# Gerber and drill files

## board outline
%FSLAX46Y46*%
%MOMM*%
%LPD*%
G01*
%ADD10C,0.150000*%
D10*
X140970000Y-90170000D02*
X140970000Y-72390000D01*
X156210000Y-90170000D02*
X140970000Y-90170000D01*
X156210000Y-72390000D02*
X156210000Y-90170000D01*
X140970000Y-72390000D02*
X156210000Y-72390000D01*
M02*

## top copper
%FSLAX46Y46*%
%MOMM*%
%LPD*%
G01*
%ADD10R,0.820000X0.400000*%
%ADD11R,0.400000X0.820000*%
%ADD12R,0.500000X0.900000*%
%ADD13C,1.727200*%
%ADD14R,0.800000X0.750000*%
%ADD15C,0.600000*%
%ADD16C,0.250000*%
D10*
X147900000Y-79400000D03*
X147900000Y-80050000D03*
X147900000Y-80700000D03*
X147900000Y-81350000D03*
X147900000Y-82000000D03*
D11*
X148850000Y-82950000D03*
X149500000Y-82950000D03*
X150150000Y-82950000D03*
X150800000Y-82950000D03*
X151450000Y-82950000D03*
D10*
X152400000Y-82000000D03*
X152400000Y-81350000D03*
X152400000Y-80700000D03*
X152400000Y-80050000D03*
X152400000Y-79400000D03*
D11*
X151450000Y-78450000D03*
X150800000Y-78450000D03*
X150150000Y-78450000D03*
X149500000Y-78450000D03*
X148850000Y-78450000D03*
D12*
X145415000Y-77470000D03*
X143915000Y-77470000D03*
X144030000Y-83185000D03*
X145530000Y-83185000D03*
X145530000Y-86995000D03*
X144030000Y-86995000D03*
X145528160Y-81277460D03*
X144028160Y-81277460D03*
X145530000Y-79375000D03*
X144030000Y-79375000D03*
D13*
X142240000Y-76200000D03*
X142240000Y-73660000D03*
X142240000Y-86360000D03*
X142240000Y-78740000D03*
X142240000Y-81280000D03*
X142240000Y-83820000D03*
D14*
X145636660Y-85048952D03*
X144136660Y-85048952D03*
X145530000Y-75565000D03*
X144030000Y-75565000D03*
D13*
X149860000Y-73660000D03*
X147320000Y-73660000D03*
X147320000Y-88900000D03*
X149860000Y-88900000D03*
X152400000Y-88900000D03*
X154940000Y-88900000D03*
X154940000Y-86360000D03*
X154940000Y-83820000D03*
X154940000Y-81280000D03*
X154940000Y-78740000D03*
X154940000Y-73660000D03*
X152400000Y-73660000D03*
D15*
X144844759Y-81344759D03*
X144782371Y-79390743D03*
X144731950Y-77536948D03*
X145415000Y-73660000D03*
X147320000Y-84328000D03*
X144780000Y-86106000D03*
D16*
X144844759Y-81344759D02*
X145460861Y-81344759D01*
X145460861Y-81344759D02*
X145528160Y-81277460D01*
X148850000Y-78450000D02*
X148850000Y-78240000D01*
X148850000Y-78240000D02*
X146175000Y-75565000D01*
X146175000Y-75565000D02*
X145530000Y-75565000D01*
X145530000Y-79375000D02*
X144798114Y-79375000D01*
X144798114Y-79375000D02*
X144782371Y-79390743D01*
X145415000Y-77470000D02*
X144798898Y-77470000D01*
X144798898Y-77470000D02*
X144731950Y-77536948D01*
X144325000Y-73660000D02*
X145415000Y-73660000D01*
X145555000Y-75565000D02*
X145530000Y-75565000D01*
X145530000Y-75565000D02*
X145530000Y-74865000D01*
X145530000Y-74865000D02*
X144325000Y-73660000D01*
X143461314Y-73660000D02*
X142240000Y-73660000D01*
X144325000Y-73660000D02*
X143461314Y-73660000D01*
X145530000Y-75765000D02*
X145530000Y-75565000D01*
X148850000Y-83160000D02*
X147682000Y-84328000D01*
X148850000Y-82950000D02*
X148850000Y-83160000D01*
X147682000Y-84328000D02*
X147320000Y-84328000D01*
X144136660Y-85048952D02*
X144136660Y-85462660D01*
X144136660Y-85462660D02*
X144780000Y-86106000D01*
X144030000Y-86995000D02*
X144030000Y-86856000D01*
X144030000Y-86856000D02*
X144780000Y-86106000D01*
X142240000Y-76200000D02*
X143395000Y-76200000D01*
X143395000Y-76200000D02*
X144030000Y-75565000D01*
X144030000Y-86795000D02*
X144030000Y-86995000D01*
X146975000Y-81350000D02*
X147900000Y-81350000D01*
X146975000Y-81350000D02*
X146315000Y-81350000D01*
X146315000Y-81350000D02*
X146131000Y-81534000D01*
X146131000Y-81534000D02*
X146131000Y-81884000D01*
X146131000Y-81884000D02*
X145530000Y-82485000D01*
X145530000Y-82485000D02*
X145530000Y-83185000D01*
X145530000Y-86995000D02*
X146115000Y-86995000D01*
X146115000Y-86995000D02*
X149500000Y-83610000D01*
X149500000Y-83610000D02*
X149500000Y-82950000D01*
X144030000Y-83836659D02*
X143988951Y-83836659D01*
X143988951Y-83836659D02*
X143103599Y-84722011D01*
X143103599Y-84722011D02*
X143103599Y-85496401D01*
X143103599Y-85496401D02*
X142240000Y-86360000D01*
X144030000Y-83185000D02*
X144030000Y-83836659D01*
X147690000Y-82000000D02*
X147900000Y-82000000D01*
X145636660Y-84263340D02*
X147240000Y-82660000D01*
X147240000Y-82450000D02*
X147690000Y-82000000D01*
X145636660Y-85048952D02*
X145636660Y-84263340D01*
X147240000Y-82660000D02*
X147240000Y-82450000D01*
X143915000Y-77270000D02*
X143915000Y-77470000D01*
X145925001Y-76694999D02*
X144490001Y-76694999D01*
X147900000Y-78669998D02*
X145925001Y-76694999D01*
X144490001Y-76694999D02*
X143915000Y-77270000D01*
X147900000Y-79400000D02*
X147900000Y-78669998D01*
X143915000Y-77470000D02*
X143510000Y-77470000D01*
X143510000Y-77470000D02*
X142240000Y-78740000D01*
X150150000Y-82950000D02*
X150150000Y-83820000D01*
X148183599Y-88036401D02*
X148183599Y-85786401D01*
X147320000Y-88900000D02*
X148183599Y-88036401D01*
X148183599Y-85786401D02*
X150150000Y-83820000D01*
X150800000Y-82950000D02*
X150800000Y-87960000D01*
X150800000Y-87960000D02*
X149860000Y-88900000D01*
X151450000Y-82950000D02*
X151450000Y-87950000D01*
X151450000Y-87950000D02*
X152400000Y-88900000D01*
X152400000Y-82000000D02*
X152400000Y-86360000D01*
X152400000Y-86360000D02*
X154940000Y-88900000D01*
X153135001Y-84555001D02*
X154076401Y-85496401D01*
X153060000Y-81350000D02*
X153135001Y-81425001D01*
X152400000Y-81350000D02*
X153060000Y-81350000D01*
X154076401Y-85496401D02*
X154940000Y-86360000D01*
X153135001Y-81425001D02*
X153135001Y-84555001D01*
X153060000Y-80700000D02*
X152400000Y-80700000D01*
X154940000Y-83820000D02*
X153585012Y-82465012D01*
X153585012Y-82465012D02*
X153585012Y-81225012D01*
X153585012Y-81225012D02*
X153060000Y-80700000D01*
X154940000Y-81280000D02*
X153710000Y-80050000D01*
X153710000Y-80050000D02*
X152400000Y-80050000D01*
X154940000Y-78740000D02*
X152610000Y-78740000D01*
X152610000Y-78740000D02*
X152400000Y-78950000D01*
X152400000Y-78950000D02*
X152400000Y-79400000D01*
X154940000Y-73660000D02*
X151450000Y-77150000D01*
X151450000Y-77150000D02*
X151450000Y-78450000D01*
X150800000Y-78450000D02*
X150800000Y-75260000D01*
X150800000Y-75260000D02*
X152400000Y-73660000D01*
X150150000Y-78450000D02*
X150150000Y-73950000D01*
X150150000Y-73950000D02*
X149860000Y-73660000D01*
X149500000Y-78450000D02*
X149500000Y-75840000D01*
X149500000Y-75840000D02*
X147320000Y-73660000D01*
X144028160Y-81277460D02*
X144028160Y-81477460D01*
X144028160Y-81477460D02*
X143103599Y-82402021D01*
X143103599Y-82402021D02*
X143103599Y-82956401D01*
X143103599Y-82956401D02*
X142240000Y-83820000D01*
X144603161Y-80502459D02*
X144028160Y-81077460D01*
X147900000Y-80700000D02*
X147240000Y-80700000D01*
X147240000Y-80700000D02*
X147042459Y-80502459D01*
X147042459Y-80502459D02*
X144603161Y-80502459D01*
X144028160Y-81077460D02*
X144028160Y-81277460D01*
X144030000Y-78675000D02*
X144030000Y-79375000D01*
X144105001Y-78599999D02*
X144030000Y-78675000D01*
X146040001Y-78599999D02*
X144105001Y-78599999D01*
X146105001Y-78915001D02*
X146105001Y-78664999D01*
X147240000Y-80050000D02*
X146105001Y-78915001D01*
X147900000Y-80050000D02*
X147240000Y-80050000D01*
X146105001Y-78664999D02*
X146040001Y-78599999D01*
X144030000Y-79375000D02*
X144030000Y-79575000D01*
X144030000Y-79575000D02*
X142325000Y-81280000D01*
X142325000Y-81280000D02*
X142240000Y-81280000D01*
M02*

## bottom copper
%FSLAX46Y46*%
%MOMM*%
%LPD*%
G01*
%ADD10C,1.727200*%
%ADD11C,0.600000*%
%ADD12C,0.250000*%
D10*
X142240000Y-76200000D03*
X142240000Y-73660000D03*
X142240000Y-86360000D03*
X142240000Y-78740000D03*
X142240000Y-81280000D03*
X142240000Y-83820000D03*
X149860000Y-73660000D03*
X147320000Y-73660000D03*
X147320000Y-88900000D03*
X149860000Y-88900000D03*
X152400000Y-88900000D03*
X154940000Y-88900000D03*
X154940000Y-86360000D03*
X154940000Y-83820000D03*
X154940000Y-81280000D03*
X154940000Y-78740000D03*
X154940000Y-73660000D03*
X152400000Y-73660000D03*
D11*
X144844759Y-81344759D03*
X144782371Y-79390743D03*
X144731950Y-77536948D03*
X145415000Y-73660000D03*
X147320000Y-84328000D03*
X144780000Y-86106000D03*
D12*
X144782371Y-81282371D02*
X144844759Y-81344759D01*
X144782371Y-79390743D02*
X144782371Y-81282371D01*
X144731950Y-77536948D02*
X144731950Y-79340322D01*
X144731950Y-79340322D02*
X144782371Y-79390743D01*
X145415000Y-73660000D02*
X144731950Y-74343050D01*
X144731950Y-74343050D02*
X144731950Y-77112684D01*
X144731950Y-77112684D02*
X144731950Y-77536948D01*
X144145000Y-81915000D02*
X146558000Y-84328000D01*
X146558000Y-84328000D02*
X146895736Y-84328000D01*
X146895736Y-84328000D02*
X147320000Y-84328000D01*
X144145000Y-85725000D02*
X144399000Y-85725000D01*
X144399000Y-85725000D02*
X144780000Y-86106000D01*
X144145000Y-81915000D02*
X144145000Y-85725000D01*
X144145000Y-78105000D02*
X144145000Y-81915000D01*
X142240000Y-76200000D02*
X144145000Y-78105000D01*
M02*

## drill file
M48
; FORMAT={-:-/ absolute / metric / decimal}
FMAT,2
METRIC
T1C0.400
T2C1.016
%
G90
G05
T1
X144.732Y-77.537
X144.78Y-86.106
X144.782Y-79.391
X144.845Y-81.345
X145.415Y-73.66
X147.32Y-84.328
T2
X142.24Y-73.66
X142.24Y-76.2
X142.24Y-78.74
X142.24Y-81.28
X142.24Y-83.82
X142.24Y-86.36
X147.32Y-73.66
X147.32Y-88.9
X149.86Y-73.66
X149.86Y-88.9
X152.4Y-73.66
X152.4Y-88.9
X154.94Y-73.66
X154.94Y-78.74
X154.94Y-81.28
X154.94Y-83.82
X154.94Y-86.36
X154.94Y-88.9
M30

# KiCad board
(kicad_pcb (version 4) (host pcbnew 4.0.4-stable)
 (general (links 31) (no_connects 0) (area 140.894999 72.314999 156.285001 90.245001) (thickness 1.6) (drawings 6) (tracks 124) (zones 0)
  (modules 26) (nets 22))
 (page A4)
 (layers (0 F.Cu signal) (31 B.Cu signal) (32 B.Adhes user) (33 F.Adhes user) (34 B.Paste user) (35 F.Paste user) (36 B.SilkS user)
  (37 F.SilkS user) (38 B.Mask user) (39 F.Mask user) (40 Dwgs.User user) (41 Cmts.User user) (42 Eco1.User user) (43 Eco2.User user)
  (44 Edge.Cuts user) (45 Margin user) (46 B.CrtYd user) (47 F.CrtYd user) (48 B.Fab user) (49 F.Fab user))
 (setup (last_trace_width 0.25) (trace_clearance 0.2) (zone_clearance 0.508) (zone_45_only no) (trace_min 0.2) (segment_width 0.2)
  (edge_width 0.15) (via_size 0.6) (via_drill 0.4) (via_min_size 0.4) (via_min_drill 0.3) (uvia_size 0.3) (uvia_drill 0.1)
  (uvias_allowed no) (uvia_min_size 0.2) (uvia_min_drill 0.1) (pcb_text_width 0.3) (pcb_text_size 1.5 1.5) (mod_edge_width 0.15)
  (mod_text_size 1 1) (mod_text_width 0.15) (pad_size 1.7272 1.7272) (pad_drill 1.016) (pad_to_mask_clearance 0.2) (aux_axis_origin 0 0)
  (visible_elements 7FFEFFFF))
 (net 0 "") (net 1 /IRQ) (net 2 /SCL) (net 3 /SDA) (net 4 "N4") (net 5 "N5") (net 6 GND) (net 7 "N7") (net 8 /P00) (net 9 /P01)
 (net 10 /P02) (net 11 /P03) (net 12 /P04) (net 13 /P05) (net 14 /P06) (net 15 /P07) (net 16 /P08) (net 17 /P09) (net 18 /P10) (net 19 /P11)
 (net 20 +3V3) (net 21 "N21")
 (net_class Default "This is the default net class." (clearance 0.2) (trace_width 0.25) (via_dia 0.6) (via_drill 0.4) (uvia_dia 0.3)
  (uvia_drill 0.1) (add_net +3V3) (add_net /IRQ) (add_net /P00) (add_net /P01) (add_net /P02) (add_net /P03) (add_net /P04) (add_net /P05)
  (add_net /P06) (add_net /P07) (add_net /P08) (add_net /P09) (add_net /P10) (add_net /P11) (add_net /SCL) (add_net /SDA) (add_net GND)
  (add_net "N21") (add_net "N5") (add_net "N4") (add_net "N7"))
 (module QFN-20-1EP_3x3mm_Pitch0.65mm (layer F.Cu) (at 150.15 80.7)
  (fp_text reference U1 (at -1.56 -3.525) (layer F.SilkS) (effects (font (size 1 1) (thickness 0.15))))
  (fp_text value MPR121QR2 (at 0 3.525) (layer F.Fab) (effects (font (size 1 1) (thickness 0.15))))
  (pad 1 smd rect (at -2.25 -1.3) (size 0.82 0.4) (layers F.Cu F.Paste F.Mask) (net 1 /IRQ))
  (pad 2 smd rect (at -2.25 -0.65) (size 0.82 0.4) (layers F.Cu F.Paste F.Mask) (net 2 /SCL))
  (pad 3 smd rect (at -2.25 0) (size 0.82 0.4) (layers F.Cu F.Paste F.Mask) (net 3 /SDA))
  (pad 4 smd rect (at -2.25 0.65) (size 0.82 0.4) (layers F.Cu F.Paste F.Mask) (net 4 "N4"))
  (pad 5 smd rect (at -2.25 1.3) (size 0.82 0.4) (layers F.Cu F.Paste F.Mask) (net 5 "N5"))
  (pad 6 smd rect (at -1.3 2.25 90) (size 0.82 0.4) (layers F.Cu F.Paste F.Mask) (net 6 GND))
  (pad 7 smd rect (at -0.65 2.25 90) (size 0.82 0.4) (layers F.Cu F.Paste F.Mask) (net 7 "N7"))
  (pad 8 smd rect (at 0 2.25 90) (size 0.82 0.4) (layers F.Cu F.Paste F.Mask) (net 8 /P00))
  (pad 9 smd rect (at 0.65 2.25 90) (size 0.82 0.4) (layers F.Cu F.Paste F.Mask) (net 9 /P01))
  (pad 10 smd rect (at 1.3 2.25 90) (size 0.82 0.4) (layers F.Cu F.Paste F.Mask) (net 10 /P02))
  (pad 11 smd rect (at 2.25 1.3) (size 0.82 0.4) (layers F.Cu F.Paste F.Mask) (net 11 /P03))
  (pad 12 smd rect (at 2.25 0.65) (size 0.82 0.4) (layers F.Cu F.Paste F.Mask) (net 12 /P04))
  (pad 13 smd rect (at 2.25 0) (size 0.82 0.4) (layers F.Cu F.Paste F.Mask) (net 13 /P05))
  (pad 14 smd rect (at 2.25 -0.65) (size 0.82 0.4) (layers F.Cu F.Paste F.Mask) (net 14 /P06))
  (pad 15 smd rect (at 2.25 -1.3) (size 0.82 0.4) (layers F.Cu F.Paste F.Mask) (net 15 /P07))
  (pad 16 smd rect (at 1.3 -2.25 90) (size 0.82 0.4) (layers F.Cu F.Paste F.Mask) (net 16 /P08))
  (pad 17 smd rect (at 0.65 -2.25 90) (size 0.82 0.4) (layers F.Cu F.Paste F.Mask) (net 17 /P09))
  (pad 18 smd rect (at 0 -2.25 90) (size 0.82 0.4) (layers F.Cu F.Paste F.Mask) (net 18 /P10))
  (pad 19 smd rect (at -0.65 -2.25 90) (size 0.82 0.4) (layers F.Cu F.Paste F.Mask) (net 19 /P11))
  (pad 20 smd rect (at -1.3 -2.25 90) (size 0.82 0.4) (layers F.Cu F.Paste F.Mask) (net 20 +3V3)))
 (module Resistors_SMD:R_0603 (layer F.Cu) (at 144.665 77.47 180)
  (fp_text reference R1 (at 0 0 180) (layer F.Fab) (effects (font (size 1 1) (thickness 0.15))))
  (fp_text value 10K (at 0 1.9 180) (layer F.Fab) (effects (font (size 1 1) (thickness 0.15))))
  (pad 1 smd rect (at -0.75 0 180) (size 0.5 0.9) (layers F.Cu F.Paste F.Mask) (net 20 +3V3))
  (pad 2 smd rect (at 0.75 0 180) (size 0.5 0.9) (layers F.Cu F.Paste F.Mask) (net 1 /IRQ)))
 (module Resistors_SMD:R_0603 (layer F.Cu) (at 144.78 83.185)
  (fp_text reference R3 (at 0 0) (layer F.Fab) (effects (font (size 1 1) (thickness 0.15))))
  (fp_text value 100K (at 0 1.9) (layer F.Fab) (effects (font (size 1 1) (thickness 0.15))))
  (pad 1 smd rect (at -0.75 0) (size 0.5 0.9) (layers F.Cu F.Paste F.Mask) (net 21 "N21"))
  (pad 2 smd rect (at 0.75 0) (size 0.5 0.9) (layers F.Cu F.Paste F.Mask) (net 4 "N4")))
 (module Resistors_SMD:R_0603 (layer F.Cu) (at 144.78 86.995 180)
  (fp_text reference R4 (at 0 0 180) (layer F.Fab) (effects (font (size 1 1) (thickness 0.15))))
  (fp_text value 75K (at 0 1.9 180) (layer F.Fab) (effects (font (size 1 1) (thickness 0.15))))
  (pad 1 smd rect (at -0.75 0 180) (size 0.5 0.9) (layers F.Cu F.Paste F.Mask) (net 7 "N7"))
  (pad 2 smd rect (at 0.75 0 180) (size 0.5 0.9) (layers F.Cu F.Paste F.Mask) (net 6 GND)))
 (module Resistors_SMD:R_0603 (layer F.Cu) (at 144.77816 81.27746 180)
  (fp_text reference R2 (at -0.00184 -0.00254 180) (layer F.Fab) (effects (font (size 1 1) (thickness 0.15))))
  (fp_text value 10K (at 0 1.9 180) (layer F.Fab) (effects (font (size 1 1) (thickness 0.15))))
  (pad 1 smd rect (at -0.75 0 180) (size 0.5 0.9) (layers F.Cu F.Paste F.Mask) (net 20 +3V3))
  (pad 2 smd rect (at 0.75 0 180) (size 0.5 0.9) (layers F.Cu F.Paste F.Mask) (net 3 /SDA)))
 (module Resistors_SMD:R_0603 (layer F.Cu) (at 144.78 79.375 180)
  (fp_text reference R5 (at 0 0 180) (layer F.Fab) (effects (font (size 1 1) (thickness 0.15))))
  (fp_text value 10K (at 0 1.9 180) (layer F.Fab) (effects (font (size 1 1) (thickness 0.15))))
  (pad 1 smd rect (at -0.75 0 180) (size 0.5 0.9) (layers F.Cu F.Paste F.Mask) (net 20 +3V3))
  (pad 2 smd rect (at 0.75 0 180) (size 0.5 0.9) (layers F.Cu F.Paste F.Mask) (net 2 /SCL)))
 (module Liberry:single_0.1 (layer F.Cu) (at 142.24 76.2)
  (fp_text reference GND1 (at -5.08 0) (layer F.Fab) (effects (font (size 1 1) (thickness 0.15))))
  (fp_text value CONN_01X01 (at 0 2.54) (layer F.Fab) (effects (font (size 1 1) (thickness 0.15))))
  (pad 1 thru_hole circle (at 0 0) (size 1.7272 1.7272) (drill 1.016) (layers *.Cu *.Mask) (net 6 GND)))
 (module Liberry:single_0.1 (layer F.Cu) (at 142.24 73.66)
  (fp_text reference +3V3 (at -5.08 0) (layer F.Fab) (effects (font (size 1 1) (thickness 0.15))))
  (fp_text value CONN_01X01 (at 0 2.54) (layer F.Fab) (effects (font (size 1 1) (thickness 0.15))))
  (pad 1 thru_hole circle (at 0 0) (size 1.7272 1.7272) (drill 1.016) (layers *.Cu *.Mask) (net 20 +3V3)))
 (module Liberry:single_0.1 (layer F.Cu) (at 142.24 86.36)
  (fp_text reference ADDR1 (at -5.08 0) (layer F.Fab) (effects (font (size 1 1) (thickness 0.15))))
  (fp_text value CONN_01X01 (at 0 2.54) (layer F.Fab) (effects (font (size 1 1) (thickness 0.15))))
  (pad 1 thru_hole circle (at 0 0) (size 1.7272 1.7272) (drill 1.016) (layers *.Cu *.Mask) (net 21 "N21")))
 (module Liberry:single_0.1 (layer F.Cu) (at 142.24 78.74)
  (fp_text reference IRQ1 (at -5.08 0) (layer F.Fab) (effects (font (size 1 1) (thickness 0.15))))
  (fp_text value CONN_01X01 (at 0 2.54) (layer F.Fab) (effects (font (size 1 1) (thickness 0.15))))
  (pad 1 thru_hole circle (at 0 0) (size 1.7272 1.7272) (drill 1.016) (layers *.Cu *.Mask) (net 1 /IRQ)))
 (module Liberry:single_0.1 (layer F.Cu) (at 142.24 81.28)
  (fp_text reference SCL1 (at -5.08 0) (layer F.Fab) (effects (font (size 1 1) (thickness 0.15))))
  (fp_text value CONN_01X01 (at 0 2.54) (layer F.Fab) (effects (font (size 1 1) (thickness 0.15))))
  (pad 1 thru_hole circle (at 0 0) (size 1.7272 1.7272) (drill 1.016) (layers *.Cu *.Mask) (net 2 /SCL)))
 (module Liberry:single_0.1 (layer F.Cu) (at 142.24 83.82)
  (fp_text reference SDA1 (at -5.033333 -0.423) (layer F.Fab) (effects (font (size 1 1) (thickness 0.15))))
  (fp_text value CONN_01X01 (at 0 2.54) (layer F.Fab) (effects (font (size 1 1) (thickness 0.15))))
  (pad 1 thru_hole circle (at 0 0) (size 1.7272 1.7272) (drill 1.016) (layers *.Cu *.Mask) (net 3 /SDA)))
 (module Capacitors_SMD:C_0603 (layer F.Cu) (at 144.88666 85.048952 180)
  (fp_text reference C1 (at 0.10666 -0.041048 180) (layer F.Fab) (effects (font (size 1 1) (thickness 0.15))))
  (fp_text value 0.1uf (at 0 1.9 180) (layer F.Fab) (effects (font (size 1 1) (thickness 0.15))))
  (pad 1 smd rect (at -0.75 0 180) (size 0.8 0.75) (layers F.Cu F.Paste F.Mask) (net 5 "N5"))
  (pad 2 smd rect (at 0.75 0 180) (size 0.8 0.75) (layers F.Cu F.Paste F.Mask) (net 6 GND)))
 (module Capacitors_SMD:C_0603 (layer F.Cu) (at 144.78 75.565 180)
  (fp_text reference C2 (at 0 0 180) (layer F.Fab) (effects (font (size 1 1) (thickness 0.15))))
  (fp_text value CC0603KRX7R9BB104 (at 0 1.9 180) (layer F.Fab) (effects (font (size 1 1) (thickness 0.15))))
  (pad 1 smd rect (at -0.75 0 180) (size 0.8 0.75) (layers F.Cu F.Paste F.Mask) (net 20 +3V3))
  (pad 2 smd rect (at 0.75 0 180) (size 0.8 0.75) (layers F.Cu F.Paste F.Mask) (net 6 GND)))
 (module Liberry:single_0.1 (layer F.Cu) (at 149.86 73.66 90)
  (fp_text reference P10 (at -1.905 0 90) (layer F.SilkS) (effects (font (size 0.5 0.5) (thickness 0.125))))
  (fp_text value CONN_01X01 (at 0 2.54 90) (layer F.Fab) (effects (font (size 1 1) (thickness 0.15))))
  (pad 1 thru_hole circle (at 0 0 90) (size 1.7272 1.7272) (drill 1.016) (layers *.Cu *.Mask) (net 18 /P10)))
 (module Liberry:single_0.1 (layer F.Cu) (at 147.32 73.66 90)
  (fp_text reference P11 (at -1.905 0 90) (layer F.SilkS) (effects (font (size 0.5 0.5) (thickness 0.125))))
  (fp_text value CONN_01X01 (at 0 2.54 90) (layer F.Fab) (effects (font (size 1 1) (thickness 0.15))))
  (pad 1 thru_hole circle (at 0 0 90) (size 1.7272 1.7272) (drill 1.016) (layers *.Cu *.Mask) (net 19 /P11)))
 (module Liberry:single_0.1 (layer F.Cu) (at 147.32 88.9 270)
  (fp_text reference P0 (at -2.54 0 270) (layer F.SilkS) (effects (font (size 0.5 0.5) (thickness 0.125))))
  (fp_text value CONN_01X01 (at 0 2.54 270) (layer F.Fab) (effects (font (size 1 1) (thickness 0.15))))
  (pad 1 thru_hole circle (at 0 0 270) (size 1.7272 1.7272) (drill 1.016) (layers *.Cu *.Mask) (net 8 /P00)))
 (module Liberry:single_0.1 (layer F.Cu) (at 149.86 88.9 270)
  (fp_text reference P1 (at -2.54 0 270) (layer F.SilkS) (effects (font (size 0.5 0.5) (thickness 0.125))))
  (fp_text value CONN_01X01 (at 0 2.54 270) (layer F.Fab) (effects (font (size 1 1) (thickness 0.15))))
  (pad 1 thru_hole circle (at 0 0 270) (size 1.7272 1.7272) (drill 1.016) (layers *.Cu *.Mask) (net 9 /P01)))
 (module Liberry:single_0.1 (layer F.Cu) (at 152.4 88.9 270)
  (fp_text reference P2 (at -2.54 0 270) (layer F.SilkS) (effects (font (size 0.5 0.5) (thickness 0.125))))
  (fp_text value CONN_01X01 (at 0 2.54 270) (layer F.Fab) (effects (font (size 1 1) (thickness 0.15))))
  (pad 1 thru_hole circle (at 0 0 270) (size 1.7272 1.7272) (drill 1.016) (layers *.Cu *.Mask) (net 10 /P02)))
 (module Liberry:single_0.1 (layer F.Cu) (at 154.94 88.9 270)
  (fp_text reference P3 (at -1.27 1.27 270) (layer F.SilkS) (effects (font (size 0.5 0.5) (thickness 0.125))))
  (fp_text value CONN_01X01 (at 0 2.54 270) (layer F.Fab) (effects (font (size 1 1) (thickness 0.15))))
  (pad 1 thru_hole circle (at 0 0 270) (size 1.7272 1.7272) (drill 1.016) (layers *.Cu *.Mask) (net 11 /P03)))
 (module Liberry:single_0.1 (layer F.Cu) (at 154.94 86.36)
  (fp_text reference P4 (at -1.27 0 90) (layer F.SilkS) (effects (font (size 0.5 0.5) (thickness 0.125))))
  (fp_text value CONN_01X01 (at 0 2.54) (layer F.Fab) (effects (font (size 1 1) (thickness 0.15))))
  (pad 1 thru_hole circle (at 0 0) (size 1.7272 1.7272) (drill 1.016) (layers *.Cu *.Mask) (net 12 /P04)))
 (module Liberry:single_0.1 (layer F.Cu) (at 154.94 83.82)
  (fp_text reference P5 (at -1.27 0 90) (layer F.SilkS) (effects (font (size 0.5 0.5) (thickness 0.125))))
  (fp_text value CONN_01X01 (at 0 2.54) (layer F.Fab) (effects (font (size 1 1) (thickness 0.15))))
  (pad 1 thru_hole circle (at 0 0) (size 1.7272 1.7272) (drill 1.016) (layers *.Cu *.Mask) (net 13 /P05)))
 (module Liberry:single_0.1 (layer F.Cu) (at 154.94 81.28 180)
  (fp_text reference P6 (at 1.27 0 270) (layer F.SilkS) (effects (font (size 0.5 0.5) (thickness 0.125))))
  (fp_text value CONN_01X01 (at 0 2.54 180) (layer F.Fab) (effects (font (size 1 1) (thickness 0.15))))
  (pad 1 thru_hole circle (at 0 0 180) (size 1.7272 1.7272) (drill 1.016) (layers *.Cu *.Mask) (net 14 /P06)))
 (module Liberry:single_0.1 (layer F.Cu) (at 154.94 78.74)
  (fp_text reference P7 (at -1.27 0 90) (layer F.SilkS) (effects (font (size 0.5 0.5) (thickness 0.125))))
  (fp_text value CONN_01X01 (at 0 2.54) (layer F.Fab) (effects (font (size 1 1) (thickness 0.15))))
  (pad 1 thru_hole circle (at 0 0) (size 1.7272 1.7272) (drill 1.016) (layers *.Cu *.Mask) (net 15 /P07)))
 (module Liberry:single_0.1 (layer F.Cu) (at 154.94 73.66 90)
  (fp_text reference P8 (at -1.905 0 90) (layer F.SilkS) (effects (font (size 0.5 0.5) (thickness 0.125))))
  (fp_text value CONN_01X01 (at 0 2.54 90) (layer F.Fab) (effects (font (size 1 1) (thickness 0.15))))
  (pad 1 thru_hole circle (at 0 0 90) (size 1.7272 1.7272) (drill 1.016) (layers *.Cu *.Mask) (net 16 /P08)))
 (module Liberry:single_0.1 (layer F.Cu) (at 152.4 73.66 90)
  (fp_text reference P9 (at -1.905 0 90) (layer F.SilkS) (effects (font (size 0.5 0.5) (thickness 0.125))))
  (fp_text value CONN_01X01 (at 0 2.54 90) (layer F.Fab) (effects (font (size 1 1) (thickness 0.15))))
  (pad 1 thru_hole circle (at 0 0 90) (size 1.7272 1.7272) (drill 1.016) (layers *.Cu *.Mask) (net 17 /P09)))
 (gr_line (start 140.97 90.17) (end 140.97 72.39) (layer Edge.Cuts) (width 0.15))
 (gr_line (start 156.21 90.17) (end 140.97 90.17) (layer Edge.Cuts) (width 0.15))
 (gr_line (start 156.21 72.39) (end 156.21 90.17) (layer Edge.Cuts) (width 0.15))
 (gr_line (start 140.97 72.39) (end 156.21 72.39) (layer Edge.Cuts) (width 0.15))
 (segment (start 144.844759 81.344759) (end 145.460861 81.344759) (width 0.25) (layer F.Cu) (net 20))
 (segment (start 145.460861 81.344759) (end 145.52816 81.27746) (width 0.25) (layer F.Cu) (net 20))
 (segment (start 148.85 78.45) (end 148.85 78.24) (width 0.25) (layer F.Cu) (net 20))
 (segment (start 148.85 78.24) (end 146.175 75.565) (width 0.25) (layer F.Cu) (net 20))
 (segment (start 146.175 75.565) (end 145.53 75.565) (width 0.25) (layer F.Cu) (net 20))
 (segment (start 144.782371 81.282371) (end 144.844759 81.344759) (width 0.25) (layer B.Cu) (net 20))
 (segment (start 144.782371 79.390743) (end 144.782371 81.282371) (width 0.25) (layer B.Cu) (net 20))
 (via (at 144.844759 81.344759) (size 0.6) (drill 0.4) (layers F.Cu B.Cu) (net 20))
 (segment (start 145.53 79.375) (end 144.798114 79.375) (width 0.25) (layer F.Cu) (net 20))
 (segment (start 144.73195 77.536948) (end 144.73195 79.340322) (width 0.25) (layer B.Cu) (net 20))
 (segment (start 144.73195 79.340322) (end 144.782371 79.390743) (width 0.25) (layer B.Cu) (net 20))
 (segment (start 144.798114 79.375) (end 144.782371 79.390743) (width 0.25) (layer F.Cu) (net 20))
 (via (at 144.782371 79.390743) (size 0.6) (drill 0.4) (layers F.Cu B.Cu) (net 20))
 (via (at 144.73195 77.536948) (size 0.6) (drill 0.4) (layers F.Cu B.Cu) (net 20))
 (segment (start 145.415 77.47) (end 144.798898 77.47) (width 0.25) (layer F.Cu) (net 20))
 (segment (start 144.798898 77.47) (end 144.73195 77.536948) (width 0.25) (layer F.Cu) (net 20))
 (segment (start 145.415 73.66) (end 144.73195 74.34305) (width 0.25) (layer B.Cu) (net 20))
 (segment (start 144.73195 74.34305) (end 144.73195 77.112684) (width 0.25) (layer B.Cu) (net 20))
 (segment (start 144.73195 77.112684) (end 144.73195 77.536948) (width 0.25) (layer B.Cu) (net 20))
 (segment (start 144.325 73.66) (end 145.415 73.66) (width 0.25) (layer F.Cu) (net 20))
 (via (at 145.415 73.66) (size 0.6) (drill 0.4) (layers F.Cu B.Cu) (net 20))
 (segment (start 145.555 75.565) (end 145.53 75.565) (width 0.25) (layer F.Cu) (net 20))
 (segment (start 145.53 75.565) (end 145.53 74.865) (width 0.25) (layer F.Cu) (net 20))
 (segment (start 145.53 74.865) (end 144.325 73.66) (width 0.25) (layer F.Cu) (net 20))
 (segment (start 143.461314 73.66) (end 142.24 73.66) (width 0.25) (layer F.Cu) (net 20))
 (segment (start 144.325 73.66) (end 143.461314 73.66) (width 0.25) (layer F.Cu) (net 20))
 (segment (start 145.53 75.765) (end 145.53 75.565) (width 0.25) (layer F.Cu) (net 20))
 (segment (start 144.145 81.915) (end 146.558 84.328) (width 0.25) (layer B.Cu) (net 6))
 (segment (start 146.558 84.328) (end 146.895736 84.328) (width 0.25) (layer B.Cu) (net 6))
 (segment (start 146.895736 84.328) (end 147.32 84.328) (width 0.25) (layer B.Cu) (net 6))
 (segment (start 148.85 83.16) (end 147.682 84.328) (width 0.25) (layer F.Cu) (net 6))
 (segment (start 148.85 82.95) (end 148.85 83.16) (width 0.25) (layer F.Cu) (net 6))
 (segment (start 147.682 84.328) (end 147.32 84.328) (width 0.25) (layer F.Cu) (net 6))
 (via (at 147.32 84.328) (size 0.6) (drill 0.4) (layers F.Cu B.Cu) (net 6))
 (segment (start 144.13666 85.048952) (end 144.13666 85.46266) (width 0.25) (layer F.Cu) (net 6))
 (segment (start 144.13666 85.46266) (end 144.78 86.106) (width 0.25) (layer F.Cu) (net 6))
 (segment (start 144.03 86.995) (end 144.03 86.856) (width 0.25) (layer F.Cu) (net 6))
 (segment (start 144.03 86.856) (end 144.78 86.106) (width 0.25) (layer F.Cu) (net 6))
 (segment (start 144.145 85.725) (end 144.399 85.725) (width 0.25) (layer B.Cu) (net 6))
 (segment (start 144.399 85.725) (end 144.78 86.106) (width 0.25) (layer B.Cu) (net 6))
 (segment (start 144.145 81.915) (end 144.145 85.725) (width 0.25) (layer B.Cu) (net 6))
 (via (at 144.78 86.106) (size 0.6) (drill 0.4) (layers F.Cu B.Cu) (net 6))
 (segment (start 144.145 78.105) (end 144.145 81.915) (width 0.25) (layer B.Cu) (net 6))
 (segment (start 142.24 76.2) (end 144.145 78.105) (width 0.25) (layer B.Cu) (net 6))
 (segment (start 142.24 76.2) (end 143.395 76.2) (width 0.25) (layer F.Cu) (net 6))
 (segment (start 143.395 76.2) (end 144.03 75.565) (width 0.25) (layer F.Cu) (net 6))
 (segment (start 144.03 86.795) (end 144.03 86.995) (width 0.25) (layer F.Cu) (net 6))
 (segment (start 146.975 81.35) (end 147.9 81.35) (width 0.25) (layer F.Cu) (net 4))
 (segment (start 146.975 81.35) (end 146.315 81.35) (width 0.25) (layer F.Cu) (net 4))
 (segment (start 146.315 81.35) (end 146.131 81.534) (width 0.25) (layer F.Cu) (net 4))
 (segment (start 146.131 81.534) (end 146.131 81.884) (width 0.25) (layer F.Cu) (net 4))
 (segment (start 146.131 81.884) (end 145.53 82.485) (width 0.25) (layer F.Cu) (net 4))
 (segment (start 145.53 82.485) (end 145.53 83.185) (width 0.25) (layer F.Cu) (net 4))
 (segment (start 145.53 86.995) (end 146.115 86.995) (width 0.25) (layer F.Cu) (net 7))
 (segment (start 146.115 86.995) (end 149.5 83.61) (width 0.25) (layer F.Cu) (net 7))
 (segment (start 149.5 83.61) (end 149.5 82.95) (width 0.25) (layer F.Cu) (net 7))
 (segment (start 144.03 83.836659) (end 143.988951 83.836659) (width 0.25) (layer F.Cu) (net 21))
 (segment (start 143.988951 83.836659) (end 143.103599 84.722011) (width 0.25) (layer F.Cu) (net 21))
 (segment (start 143.103599 84.722011) (end 143.103599 85.496401) (width 0.25) (layer F.Cu) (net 21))
 (segment (start 143.103599 85.496401) (end 142.24 86.36) (width 0.25) (layer F.Cu) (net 21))
 (segment (start 144.03 83.185) (end 144.03 83.836659) (width 0.25) (layer F.Cu) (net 21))
 (segment (start 147.69 82) (end 147.9 82) (width 0.25) (layer F.Cu) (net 5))
 (segment (start 145.63666 84.26334) (end 147.24 82.66) (width 0.25) (layer F.Cu) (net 5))
 (segment (start 147.24 82.45) (end 147.69 82) (width 0.25) (layer F.Cu) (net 5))
 (segment (start 145.63666 85.048952) (end 145.63666 84.26334) (width 0.25) (layer F.Cu) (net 5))
 (segment (start 147.24 82.66) (end 147.24 82.45) (width 0.25) (layer F.Cu) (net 5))
 (segment (start 143.915 77.27) (end 143.915 77.47) (width 0.25) (layer F.Cu) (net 1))
 (segment (start 145.925001 76.694999) (end 144.490001 76.694999) (width 0.25) (layer F.Cu) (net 1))
 (segment (start 147.9 78.669998) (end 145.925001 76.694999) (width 0.25) (layer F.Cu) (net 1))
 (segment (start 144.490001 76.694999) (end 143.915 77.27) (width 0.25) (layer F.Cu) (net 1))
 (segment (start 147.9 79.4) (end 147.9 78.669998) (width 0.25) (layer F.Cu) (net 1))
 (segment (start 143.915 77.47) (end 143.51 77.47) (width 0.25) (layer F.Cu) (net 1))
 (segment (start 143.51 77.47) (end 142.24 78.74) (width 0.25) (layer F.Cu) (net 1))
 (segment (start 150.15 82.95) (end 150.15 83.82) (width 0.25) (layer F.Cu) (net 8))
 (segment (start 148.183599 88.036401) (end 148.183599 85.786401) (width 0.25) (layer F.Cu) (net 8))
 (segment (start 147.32 88.9) (end 148.183599 88.036401) (width 0.25) (layer F.Cu) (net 8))
 (segment (start 148.183599 85.786401) (end 150.15 83.82) (width 0.25) (layer F.Cu) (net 8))
 (segment (start 150.8 82.95) (end 150.8 87.96) (width 0.25) (layer F.Cu) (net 9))
 (segment (start 150.8 87.96) (end 149.86 88.9) (width 0.25) (layer F.Cu) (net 9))
 (segment (start 151.45 82.95) (end 151.45 87.95) (width 0.25) (layer F.Cu) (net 10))
 (segment (start 151.45 87.95) (end 152.4 88.9) (width 0.25) (layer F.Cu) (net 10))
 (segment (start 152.4 82) (end 152.4 86.36) (width 0.25) (layer F.Cu) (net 11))
 (segment (start 152.4 86.36) (end 154.94 88.9) (width 0.25) (layer F.Cu) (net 11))
 (segment (start 153.135001 84.555001) (end 154.076401 85.496401) (width 0.25) (layer F.Cu) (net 12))
 (segment (start 153.06 81.35) (end 153.135001 81.425001) (width 0.25) (layer F.Cu) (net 12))
 (segment (start 152.4 81.35) (end 153.06 81.35) (width 0.25) (layer F.Cu) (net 12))
 (segment (start 154.076401 85.496401) (end 154.94 86.36) (width 0.25) (layer F.Cu) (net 12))
 (segment (start 153.135001 81.425001) (end 153.135001 84.555001) (width 0.25) (layer F.Cu) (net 12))
 (segment (start 153.06 80.7) (end 152.4 80.7) (width 0.25) (layer F.Cu) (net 13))
 (segment (start 154.94 83.82) (end 153.585012 82.465012) (width 0.25) (layer F.Cu) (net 13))
 (segment (start 153.585012 82.465012) (end 153.585012 81.225012) (width 0.25) (layer F.Cu) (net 13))
 (segment (start 153.585012 81.225012) (end 153.06 80.7) (width 0.25) (layer F.Cu) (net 13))
 (segment (start 154.94 81.28) (end 153.71 80.05) (width 0.25) (layer F.Cu) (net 14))
 (segment (start 153.71 80.05) (end 152.4 80.05) (width 0.25) (layer F.Cu) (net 14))
 (segment (start 154.94 78.74) (end 152.61 78.74) (width 0.25) (layer F.Cu) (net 15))
 (segment (start 152.61 78.74) (end 152.4 78.95) (width 0.25) (layer F.Cu) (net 15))
 (segment (start 152.4 78.95) (end 152.4 79.4) (width 0.25) (layer F.Cu) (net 15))
 (segment (start 154.94 73.66) (end 151.45 77.15) (width 0.25) (layer F.Cu) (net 16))
 (segment (start 151.45 77.15) (end 151.45 78.45) (width 0.25) (layer F.Cu) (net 16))
 (segment (start 150.8 78.45) (end 150.8 75.26) (width 0.25) (layer F.Cu) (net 17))
 (segment (start 150.8 75.26) (end 152.4 73.66) (width 0.25) (layer F.Cu) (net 17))
 (segment (start 150.15 78.45) (end 150.15 73.95) (width 0.25) (layer F.Cu) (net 18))
 (segment (start 150.15 73.95) (end 149.86 73.66) (width 0.25) (layer F.Cu) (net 18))
 (segment (start 149.5 78.45) (end 149.5 75.84) (width 0.25) (layer F.Cu) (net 19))
 (segment (start 149.5 75.84) (end 147.32 73.66) (width 0.25) (layer F.Cu) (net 19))
 (segment (start 144.02816 81.27746) (end 144.02816 81.47746) (width 0.25) (layer F.Cu) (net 3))
 (segment (start 144.02816 81.47746) (end 143.103599 82.402021) (width 0.25) (layer F.Cu) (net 3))
 (segment (start 143.103599 82.402021) (end 143.103599 82.956401) (width 0.25) (layer F.Cu) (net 3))
 (segment (start 143.103599 82.956401) (end 142.24 83.82) (width 0.25) (layer F.Cu) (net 3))
 (segment (start 144.603161 80.502459) (end 144.02816 81.07746) (width 0.25) (layer F.Cu) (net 3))
 (segment (start 147.9 80.7) (end 147.24 80.7) (width 0.25) (layer F.Cu) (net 3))
 (segment (start 147.24 80.7) (end 147.042459 80.502459) (width 0.25) (layer F.Cu) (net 3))
 (segment (start 147.042459 80.502459) (end 144.603161 80.502459) (width 0.25) (layer F.Cu) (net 3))
 (segment (start 144.02816 81.07746) (end 144.02816 81.27746) (width 0.25) (layer F.Cu) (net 3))
 (segment (start 144.03 78.675) (end 144.03 79.375) (width 0.25) (layer F.Cu) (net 2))
 (segment (start 144.105001 78.599999) (end 144.03 78.675) (width 0.25) (layer F.Cu) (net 2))
 (segment (start 146.040001 78.599999) (end 144.105001 78.599999) (width 0.25) (layer F.Cu) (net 2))
 (segment (start 146.105001 78.915001) (end 146.105001 78.664999) (width 0.25) (layer F.Cu) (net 2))
 (segment (start 147.24 80.05) (end 146.105001 78.915001) (width 0.25) (layer F.Cu) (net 2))
 (segment (start 147.9 80.05) (end 147.24 80.05) (width 0.25) (layer F.Cu) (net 2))
 (segment (start 146.105001 78.664999) (end 146.040001 78.599999) (width 0.25) (layer F.Cu) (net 2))
 (segment (start 144.03 79.375) (end 144.03 79.575) (width 0.25) (layer F.Cu) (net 2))
 (segment (start 144.03 79.575) (end 142.325 81.28) (width 0.25) (layer F.Cu) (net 2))
 (segment (start 142.325 81.28) (end 142.24 81.28) (width 0.25) (layer F.Cu) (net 2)))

